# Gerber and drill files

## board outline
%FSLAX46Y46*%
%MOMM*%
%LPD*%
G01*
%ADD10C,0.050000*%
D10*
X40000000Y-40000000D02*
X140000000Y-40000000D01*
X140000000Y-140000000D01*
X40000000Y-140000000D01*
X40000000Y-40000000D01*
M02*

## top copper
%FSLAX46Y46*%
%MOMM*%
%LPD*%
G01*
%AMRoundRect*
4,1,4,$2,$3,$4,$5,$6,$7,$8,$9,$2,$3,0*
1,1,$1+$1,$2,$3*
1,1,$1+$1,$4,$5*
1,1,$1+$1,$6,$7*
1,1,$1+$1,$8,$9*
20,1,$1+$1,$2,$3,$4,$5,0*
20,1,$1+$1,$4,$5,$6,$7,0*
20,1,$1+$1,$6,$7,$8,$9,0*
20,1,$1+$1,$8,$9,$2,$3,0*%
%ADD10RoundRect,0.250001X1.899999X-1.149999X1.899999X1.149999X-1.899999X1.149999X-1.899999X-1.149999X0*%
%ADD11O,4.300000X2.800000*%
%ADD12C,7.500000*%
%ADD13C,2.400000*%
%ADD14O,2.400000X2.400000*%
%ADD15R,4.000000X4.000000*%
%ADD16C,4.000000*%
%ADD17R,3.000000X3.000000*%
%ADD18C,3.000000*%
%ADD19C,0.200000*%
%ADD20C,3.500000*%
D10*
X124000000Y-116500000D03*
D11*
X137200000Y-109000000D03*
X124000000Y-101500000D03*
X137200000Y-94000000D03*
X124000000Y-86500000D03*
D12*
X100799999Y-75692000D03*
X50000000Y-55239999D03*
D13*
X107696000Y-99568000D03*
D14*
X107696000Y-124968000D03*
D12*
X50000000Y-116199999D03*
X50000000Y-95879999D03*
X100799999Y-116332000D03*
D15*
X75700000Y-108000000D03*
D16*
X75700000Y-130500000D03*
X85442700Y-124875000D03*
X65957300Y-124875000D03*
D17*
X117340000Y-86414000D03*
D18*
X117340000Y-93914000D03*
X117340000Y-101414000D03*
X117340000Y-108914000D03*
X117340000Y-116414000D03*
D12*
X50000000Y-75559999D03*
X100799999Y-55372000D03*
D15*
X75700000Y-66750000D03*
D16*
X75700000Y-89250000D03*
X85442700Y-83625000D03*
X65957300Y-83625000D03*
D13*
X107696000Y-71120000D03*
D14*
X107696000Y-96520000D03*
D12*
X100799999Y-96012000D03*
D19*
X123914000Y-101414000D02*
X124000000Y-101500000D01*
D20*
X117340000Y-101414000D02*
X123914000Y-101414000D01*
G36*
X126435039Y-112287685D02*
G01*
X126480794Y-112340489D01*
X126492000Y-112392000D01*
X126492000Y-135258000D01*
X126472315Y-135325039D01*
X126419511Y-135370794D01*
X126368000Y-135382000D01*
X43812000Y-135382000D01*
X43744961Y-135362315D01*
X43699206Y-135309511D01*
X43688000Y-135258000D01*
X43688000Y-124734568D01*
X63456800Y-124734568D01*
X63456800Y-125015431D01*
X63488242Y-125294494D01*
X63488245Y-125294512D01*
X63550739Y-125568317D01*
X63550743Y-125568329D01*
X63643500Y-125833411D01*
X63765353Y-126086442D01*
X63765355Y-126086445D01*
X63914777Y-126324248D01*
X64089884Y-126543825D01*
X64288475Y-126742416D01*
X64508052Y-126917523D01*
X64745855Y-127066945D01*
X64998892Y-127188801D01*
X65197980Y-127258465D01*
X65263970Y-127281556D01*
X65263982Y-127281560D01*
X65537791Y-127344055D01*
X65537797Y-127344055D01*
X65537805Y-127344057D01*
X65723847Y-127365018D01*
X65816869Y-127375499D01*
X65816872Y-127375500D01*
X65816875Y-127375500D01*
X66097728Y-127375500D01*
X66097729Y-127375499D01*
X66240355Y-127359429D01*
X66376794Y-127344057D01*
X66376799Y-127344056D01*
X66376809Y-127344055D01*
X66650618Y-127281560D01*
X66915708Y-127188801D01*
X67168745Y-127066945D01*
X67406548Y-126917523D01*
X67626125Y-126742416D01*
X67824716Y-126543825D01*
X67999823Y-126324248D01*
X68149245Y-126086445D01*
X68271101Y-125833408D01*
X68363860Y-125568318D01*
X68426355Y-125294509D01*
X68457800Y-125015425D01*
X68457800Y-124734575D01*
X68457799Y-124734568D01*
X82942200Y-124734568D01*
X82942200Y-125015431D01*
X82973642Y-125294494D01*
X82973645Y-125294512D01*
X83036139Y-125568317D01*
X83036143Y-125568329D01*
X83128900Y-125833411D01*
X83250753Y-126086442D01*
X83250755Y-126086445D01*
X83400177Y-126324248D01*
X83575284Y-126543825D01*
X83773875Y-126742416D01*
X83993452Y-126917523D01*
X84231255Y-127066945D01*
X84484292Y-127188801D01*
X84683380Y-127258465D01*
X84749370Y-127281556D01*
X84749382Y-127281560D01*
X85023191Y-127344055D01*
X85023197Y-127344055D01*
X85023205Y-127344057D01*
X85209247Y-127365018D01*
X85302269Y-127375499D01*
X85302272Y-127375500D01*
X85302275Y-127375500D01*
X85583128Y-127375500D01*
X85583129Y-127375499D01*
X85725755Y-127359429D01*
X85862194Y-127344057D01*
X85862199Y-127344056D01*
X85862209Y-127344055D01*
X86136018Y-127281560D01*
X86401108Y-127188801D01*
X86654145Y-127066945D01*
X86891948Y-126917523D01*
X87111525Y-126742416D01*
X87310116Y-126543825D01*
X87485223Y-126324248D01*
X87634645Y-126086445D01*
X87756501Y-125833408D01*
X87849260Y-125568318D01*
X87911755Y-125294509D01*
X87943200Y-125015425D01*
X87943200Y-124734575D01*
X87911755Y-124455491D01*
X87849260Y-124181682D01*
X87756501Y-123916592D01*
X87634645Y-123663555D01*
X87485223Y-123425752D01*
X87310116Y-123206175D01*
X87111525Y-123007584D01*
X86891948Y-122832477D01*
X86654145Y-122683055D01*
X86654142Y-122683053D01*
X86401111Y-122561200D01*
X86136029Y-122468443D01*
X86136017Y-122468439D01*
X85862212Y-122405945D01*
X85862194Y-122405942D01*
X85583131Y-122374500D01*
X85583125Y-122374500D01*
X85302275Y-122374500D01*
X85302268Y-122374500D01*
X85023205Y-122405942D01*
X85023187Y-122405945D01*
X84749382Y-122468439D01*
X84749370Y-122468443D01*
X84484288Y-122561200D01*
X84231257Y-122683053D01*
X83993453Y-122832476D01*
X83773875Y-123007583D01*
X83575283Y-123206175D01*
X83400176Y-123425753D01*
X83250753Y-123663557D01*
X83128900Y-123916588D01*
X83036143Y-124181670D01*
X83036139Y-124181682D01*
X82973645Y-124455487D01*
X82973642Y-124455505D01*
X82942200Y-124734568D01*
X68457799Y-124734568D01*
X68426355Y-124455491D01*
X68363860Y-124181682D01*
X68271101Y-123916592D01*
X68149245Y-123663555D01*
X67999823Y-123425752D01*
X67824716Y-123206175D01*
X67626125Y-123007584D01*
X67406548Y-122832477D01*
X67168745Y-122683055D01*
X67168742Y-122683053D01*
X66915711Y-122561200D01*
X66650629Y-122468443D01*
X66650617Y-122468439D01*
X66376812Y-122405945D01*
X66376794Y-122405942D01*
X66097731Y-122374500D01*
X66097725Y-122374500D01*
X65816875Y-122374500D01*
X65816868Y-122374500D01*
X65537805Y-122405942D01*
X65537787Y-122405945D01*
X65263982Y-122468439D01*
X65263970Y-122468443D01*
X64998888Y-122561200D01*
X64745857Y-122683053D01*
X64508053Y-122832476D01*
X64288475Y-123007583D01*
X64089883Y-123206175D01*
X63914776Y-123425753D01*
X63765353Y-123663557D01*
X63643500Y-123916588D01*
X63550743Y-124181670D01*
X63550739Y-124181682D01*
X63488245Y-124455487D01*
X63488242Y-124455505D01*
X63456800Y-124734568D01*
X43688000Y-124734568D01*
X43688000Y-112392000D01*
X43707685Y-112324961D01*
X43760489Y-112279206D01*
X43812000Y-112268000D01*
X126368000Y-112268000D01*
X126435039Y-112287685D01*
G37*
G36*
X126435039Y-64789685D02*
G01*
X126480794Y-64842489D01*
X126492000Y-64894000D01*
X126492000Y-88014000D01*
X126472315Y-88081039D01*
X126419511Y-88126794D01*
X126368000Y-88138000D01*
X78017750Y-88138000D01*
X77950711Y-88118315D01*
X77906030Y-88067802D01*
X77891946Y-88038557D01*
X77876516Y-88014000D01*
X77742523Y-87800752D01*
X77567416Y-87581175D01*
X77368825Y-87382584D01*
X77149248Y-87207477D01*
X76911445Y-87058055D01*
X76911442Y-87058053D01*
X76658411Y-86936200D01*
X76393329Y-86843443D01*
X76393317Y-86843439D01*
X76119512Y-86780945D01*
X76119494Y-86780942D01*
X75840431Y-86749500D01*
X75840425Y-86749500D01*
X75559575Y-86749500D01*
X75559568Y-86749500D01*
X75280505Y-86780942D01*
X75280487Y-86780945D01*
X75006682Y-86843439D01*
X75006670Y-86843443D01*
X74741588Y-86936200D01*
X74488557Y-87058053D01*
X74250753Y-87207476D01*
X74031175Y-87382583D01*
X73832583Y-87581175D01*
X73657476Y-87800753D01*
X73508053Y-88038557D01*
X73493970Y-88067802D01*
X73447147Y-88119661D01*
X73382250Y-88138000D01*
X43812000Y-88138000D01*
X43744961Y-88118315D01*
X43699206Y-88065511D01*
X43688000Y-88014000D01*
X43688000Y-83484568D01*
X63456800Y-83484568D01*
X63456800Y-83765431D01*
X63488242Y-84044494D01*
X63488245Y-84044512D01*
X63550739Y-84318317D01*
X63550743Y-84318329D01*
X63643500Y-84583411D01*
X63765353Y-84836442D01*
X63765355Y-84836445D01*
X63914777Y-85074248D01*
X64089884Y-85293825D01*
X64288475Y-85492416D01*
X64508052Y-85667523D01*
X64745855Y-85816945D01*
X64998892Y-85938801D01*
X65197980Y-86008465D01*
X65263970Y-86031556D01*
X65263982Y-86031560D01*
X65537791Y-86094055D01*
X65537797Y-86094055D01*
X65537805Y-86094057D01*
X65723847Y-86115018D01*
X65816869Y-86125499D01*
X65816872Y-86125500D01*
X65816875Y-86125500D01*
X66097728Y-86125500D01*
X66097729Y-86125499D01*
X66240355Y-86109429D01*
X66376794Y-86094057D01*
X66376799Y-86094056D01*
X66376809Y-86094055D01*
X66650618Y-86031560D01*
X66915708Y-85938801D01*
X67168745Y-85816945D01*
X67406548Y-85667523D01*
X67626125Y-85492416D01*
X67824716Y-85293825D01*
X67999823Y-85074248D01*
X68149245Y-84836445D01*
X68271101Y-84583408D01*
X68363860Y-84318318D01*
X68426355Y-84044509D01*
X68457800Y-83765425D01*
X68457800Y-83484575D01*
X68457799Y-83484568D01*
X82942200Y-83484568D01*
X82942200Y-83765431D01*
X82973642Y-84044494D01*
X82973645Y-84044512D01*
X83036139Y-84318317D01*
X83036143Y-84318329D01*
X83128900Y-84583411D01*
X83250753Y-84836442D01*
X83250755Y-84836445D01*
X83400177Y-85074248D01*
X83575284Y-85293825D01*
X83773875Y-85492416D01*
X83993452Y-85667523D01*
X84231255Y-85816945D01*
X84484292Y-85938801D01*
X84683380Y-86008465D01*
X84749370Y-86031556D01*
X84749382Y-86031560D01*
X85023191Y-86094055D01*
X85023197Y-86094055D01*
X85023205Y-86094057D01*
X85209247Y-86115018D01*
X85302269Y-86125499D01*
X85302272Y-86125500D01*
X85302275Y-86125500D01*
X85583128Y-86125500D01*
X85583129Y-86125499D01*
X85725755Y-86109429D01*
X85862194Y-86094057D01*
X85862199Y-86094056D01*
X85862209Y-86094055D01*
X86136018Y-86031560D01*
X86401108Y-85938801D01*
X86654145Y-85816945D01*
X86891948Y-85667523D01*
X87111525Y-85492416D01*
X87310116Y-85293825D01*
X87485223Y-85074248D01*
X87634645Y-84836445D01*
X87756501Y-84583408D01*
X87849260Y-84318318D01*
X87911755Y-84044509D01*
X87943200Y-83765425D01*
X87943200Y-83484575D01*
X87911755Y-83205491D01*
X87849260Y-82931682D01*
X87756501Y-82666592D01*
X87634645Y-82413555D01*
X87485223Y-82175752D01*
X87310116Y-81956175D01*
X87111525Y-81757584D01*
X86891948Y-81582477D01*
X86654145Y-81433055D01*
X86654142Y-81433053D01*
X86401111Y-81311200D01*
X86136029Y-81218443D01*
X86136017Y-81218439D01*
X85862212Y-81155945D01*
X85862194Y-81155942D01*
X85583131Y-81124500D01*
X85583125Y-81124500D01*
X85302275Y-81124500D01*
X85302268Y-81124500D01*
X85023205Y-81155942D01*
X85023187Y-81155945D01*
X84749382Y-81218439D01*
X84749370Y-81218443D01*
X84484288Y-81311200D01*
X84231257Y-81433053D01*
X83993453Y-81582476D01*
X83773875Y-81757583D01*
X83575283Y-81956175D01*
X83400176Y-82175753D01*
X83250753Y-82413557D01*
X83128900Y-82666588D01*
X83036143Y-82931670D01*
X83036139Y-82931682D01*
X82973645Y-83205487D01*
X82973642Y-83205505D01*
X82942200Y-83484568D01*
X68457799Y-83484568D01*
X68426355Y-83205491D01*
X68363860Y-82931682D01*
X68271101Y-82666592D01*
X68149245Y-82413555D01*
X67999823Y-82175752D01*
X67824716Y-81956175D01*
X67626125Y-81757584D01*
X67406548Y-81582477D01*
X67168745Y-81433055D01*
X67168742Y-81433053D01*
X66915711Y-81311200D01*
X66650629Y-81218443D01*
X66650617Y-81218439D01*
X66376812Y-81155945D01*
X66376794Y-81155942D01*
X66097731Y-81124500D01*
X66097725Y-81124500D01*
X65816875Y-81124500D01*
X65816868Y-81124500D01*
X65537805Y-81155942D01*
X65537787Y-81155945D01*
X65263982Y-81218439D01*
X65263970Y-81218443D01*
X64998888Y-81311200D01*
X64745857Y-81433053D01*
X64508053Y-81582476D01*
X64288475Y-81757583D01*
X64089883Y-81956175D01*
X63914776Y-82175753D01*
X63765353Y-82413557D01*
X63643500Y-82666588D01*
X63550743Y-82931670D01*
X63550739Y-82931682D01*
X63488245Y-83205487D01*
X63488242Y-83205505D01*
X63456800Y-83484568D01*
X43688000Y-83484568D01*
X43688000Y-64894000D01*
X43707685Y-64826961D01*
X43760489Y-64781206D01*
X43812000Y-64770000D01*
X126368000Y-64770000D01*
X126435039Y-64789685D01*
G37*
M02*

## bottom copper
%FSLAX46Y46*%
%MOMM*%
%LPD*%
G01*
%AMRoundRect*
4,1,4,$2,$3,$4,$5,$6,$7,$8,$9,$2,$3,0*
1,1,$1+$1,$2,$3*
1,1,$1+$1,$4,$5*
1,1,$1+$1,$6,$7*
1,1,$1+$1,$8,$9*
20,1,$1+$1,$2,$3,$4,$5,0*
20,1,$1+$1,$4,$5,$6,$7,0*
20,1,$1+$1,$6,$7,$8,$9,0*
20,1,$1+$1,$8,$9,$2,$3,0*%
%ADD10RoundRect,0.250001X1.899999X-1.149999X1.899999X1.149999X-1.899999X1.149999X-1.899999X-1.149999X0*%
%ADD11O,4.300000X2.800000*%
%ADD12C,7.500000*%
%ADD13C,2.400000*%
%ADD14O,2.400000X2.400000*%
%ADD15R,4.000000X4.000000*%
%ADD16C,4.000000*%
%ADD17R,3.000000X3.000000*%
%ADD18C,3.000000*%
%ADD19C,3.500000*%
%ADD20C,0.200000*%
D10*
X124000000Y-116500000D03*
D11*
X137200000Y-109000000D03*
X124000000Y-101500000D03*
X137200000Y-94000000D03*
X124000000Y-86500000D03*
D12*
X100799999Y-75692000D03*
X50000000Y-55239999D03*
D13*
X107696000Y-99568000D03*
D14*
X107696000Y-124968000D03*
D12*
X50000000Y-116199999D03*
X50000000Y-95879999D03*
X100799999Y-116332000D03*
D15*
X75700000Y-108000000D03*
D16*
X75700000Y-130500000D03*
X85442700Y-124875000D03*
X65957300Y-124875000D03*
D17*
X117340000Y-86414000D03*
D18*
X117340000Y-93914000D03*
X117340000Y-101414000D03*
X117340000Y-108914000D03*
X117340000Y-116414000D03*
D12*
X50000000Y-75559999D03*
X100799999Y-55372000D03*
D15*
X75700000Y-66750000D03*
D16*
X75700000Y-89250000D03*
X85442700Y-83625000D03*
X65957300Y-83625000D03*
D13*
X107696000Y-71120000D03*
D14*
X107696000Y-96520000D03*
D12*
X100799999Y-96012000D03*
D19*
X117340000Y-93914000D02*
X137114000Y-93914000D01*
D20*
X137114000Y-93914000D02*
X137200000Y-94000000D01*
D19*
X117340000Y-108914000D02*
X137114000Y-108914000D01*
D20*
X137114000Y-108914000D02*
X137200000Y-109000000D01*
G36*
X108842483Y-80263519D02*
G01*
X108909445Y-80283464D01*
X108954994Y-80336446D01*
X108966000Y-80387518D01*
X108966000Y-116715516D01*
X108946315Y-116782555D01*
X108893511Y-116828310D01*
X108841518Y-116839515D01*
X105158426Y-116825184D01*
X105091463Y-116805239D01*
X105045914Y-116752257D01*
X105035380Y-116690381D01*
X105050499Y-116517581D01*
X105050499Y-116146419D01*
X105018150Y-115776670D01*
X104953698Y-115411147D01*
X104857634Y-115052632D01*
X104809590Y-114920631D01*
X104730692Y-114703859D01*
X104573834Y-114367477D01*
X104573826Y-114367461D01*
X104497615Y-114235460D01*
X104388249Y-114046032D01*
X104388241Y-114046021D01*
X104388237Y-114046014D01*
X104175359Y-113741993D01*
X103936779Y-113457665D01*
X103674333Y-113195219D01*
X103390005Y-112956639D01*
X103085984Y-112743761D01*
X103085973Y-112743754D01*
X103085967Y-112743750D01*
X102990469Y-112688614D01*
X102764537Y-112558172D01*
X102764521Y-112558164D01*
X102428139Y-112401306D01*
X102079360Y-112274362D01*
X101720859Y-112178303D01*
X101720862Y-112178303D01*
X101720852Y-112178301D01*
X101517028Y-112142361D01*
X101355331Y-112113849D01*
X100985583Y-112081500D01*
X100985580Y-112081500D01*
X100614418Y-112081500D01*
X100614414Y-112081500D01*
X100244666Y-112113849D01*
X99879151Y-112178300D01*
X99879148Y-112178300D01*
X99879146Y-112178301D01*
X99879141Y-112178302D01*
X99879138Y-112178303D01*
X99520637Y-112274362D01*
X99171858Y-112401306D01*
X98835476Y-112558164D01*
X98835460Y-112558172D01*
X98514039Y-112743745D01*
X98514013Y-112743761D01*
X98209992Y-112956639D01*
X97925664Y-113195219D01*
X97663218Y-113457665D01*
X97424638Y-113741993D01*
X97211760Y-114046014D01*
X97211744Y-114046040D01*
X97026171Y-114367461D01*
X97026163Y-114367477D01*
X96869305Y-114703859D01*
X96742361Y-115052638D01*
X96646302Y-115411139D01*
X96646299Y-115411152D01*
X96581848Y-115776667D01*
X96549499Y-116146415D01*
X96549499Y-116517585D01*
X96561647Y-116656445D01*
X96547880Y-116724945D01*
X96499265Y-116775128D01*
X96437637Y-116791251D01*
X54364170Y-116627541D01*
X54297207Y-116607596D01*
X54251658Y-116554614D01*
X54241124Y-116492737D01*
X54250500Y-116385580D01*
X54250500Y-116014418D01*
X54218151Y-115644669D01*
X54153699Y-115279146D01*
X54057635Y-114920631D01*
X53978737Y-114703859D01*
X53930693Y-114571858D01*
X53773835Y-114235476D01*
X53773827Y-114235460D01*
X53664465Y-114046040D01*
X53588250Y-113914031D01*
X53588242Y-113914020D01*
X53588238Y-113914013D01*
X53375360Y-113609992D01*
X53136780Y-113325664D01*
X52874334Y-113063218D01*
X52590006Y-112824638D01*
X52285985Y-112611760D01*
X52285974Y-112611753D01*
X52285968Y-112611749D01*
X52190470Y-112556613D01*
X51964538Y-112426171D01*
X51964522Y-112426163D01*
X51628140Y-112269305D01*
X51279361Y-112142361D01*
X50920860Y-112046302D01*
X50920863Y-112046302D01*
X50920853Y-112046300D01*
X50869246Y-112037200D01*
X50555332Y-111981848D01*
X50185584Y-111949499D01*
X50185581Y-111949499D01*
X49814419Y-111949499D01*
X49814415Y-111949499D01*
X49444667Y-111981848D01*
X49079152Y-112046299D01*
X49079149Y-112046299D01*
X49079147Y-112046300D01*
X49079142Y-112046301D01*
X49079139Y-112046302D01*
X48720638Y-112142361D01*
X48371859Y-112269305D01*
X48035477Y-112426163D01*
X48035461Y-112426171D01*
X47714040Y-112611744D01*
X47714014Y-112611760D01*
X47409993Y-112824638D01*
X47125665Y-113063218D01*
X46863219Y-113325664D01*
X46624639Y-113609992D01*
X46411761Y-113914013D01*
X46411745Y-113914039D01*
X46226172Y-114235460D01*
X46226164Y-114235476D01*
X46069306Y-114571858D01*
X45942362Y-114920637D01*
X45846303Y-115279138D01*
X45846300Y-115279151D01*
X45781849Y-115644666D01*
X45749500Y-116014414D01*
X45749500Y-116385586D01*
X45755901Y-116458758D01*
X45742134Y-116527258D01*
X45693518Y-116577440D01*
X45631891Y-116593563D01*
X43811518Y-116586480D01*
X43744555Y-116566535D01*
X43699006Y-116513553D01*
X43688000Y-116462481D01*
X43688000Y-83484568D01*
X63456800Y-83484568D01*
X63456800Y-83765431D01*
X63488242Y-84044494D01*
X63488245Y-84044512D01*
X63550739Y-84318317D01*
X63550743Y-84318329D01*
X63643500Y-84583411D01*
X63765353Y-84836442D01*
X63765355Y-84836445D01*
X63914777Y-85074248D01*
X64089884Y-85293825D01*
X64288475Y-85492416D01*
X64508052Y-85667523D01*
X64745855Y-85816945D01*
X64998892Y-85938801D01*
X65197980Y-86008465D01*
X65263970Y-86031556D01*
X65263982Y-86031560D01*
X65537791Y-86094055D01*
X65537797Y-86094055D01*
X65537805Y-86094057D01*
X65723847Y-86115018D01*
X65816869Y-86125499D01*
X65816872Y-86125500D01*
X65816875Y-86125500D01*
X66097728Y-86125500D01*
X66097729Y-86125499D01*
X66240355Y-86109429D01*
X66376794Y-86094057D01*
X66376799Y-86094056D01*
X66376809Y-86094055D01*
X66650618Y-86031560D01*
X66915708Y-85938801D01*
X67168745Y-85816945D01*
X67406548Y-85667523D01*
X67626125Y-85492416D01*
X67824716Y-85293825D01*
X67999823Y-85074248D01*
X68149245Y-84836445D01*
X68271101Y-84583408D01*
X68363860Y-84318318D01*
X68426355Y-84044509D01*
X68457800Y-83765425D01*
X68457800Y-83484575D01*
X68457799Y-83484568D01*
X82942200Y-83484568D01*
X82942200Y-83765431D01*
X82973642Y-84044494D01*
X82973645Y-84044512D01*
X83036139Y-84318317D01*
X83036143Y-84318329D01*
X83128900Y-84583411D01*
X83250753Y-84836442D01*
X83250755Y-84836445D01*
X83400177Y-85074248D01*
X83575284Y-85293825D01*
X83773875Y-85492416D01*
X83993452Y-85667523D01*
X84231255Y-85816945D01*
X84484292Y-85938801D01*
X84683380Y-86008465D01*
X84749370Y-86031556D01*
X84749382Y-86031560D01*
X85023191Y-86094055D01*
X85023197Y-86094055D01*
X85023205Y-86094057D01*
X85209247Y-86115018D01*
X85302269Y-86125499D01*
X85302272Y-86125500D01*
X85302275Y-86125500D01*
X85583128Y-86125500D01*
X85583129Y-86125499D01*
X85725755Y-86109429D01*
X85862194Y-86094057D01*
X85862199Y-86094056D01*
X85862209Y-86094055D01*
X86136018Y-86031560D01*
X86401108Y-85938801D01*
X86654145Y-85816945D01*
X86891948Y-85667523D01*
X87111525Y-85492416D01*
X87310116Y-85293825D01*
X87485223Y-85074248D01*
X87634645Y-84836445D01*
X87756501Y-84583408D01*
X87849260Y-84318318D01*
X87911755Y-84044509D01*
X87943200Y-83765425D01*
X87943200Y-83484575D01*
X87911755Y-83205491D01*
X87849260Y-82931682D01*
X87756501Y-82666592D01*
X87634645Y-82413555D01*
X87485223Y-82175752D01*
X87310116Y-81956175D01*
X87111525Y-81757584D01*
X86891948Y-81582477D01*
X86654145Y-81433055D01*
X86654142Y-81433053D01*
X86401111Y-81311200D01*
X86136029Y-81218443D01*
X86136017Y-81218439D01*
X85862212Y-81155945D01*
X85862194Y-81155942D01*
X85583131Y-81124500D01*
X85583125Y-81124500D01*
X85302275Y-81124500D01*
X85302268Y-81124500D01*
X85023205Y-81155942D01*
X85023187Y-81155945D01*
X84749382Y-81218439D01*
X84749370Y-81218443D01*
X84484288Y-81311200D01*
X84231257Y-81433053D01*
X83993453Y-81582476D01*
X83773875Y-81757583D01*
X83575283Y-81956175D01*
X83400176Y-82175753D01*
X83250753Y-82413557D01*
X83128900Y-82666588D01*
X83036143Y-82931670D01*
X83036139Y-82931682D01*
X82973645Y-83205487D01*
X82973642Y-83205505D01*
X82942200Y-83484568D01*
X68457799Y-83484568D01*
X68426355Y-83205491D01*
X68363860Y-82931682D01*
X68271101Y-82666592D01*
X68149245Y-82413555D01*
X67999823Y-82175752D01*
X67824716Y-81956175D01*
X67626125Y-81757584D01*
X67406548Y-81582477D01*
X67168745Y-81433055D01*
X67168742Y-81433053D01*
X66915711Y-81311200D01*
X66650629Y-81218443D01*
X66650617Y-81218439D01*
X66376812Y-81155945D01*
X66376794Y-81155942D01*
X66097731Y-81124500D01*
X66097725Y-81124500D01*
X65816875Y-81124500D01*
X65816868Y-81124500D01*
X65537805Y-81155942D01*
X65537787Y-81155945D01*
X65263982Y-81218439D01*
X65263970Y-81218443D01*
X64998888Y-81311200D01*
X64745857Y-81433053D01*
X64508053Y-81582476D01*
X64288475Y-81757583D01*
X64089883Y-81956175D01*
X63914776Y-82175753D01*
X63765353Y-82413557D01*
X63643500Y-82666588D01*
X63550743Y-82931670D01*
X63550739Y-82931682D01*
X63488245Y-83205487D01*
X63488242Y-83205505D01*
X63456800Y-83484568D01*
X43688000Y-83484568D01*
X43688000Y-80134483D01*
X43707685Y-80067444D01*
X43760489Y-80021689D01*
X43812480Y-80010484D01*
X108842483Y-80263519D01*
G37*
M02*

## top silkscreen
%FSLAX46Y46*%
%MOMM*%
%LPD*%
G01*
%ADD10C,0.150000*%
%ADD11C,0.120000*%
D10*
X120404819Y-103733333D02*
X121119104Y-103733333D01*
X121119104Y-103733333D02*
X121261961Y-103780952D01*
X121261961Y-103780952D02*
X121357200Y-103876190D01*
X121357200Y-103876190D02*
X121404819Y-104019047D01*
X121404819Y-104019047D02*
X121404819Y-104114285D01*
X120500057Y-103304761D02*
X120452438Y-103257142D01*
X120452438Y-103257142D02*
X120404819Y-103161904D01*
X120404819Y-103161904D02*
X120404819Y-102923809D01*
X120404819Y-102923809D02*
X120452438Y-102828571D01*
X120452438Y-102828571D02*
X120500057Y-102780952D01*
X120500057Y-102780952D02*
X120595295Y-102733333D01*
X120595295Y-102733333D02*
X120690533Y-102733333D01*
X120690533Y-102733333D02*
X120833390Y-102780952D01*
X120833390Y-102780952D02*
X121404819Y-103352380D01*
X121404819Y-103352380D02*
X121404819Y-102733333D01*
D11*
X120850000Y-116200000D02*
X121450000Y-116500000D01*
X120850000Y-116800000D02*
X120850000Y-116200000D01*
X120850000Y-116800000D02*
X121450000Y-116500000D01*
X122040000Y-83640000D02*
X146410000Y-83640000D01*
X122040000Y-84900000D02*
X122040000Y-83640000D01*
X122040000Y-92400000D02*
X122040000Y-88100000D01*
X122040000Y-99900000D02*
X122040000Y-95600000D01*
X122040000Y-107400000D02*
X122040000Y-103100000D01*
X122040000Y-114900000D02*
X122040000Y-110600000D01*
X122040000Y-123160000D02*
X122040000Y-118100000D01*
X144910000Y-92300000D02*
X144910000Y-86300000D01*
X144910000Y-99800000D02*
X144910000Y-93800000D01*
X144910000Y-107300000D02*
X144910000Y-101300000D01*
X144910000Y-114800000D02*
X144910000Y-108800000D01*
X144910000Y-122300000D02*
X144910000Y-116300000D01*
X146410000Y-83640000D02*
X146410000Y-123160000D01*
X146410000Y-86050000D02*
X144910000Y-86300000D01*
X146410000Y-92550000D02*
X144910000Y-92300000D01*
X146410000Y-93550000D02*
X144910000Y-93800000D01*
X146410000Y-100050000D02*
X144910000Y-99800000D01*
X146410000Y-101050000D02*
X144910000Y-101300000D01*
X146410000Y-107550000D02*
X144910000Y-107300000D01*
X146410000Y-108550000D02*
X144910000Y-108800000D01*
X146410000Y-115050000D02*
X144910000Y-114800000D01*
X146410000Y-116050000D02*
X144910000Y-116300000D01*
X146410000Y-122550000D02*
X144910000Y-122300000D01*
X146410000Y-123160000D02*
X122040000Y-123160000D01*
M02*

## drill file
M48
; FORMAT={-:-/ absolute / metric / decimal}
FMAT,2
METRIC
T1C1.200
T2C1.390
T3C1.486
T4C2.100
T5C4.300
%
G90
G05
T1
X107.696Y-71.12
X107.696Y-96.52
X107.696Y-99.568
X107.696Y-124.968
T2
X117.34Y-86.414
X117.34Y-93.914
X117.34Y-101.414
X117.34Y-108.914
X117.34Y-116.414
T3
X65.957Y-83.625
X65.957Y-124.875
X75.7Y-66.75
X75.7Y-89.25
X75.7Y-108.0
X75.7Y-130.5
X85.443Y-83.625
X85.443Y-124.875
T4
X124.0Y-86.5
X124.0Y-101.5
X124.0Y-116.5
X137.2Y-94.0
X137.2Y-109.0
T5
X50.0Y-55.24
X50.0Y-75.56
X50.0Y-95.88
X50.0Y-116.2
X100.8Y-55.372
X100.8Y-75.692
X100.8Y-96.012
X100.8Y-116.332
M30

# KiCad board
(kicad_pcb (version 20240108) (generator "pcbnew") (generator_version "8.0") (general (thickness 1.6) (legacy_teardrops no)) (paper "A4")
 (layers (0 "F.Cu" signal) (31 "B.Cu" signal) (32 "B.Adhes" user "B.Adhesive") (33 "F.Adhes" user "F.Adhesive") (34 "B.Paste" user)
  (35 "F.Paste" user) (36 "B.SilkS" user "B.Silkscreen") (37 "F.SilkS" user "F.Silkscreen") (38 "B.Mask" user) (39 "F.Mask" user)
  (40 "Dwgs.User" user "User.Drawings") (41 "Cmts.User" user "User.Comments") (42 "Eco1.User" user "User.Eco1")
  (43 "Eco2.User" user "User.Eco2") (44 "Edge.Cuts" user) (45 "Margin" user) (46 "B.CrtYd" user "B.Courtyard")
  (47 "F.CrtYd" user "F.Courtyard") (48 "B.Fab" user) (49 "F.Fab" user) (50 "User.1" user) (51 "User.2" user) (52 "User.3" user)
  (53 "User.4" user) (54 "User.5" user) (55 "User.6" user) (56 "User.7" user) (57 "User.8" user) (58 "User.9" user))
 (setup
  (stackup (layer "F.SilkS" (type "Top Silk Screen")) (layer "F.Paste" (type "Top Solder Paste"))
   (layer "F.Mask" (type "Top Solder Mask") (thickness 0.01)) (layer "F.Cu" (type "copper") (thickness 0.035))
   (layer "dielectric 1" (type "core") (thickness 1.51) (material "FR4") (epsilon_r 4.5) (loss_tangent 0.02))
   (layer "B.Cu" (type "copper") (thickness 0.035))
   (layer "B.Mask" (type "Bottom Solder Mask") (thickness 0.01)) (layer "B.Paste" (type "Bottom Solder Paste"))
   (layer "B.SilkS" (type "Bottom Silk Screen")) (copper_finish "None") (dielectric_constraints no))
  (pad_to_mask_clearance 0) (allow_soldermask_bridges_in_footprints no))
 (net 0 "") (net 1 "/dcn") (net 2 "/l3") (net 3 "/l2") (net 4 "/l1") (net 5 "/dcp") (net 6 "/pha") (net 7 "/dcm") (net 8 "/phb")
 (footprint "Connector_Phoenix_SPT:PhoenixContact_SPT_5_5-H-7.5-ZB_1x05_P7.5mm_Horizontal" (layer "F.Cu") (at 124 116.5 90)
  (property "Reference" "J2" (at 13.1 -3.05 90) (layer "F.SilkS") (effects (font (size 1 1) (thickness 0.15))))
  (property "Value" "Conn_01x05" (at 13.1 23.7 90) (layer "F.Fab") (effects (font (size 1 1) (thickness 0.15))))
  (fp_line (start 0.3 -3.15) (end 0 -2.55) (stroke (width 0.12) (type solid)) (layer "F.SilkS"))
  (fp_line (start -0.3 -3.15) (end 0.3 -3.15) (stroke (width 0.12) (type solid)) (layer "F.SilkS"))
  (fp_line (start -0.3 -3.15) (end 0 -2.55) (stroke (width 0.12) (type solid)) (layer "F.SilkS"))
  (fp_line (start 32.86 -1.96) (end 32.86 22.41) (stroke (width 0.12) (type solid)) (layer "F.SilkS"))
  (fp_line (start 31.6 -1.96) (end 32.86 -1.96) (stroke (width 0.12) (type solid)) (layer "F.SilkS"))
  (fp_line (start 24.1 -1.96) (end 28.4 -1.96) (stroke (width 0.12) (type solid)) (layer "F.SilkS"))
  (fp_line (start 16.6 -1.96) (end 20.9 -1.96) (stroke (width 0.12) (type solid)) (layer "F.SilkS"))
  (fp_line (start 9.1 -1.96) (end 13.4 -1.96) (stroke (width 0.12) (type solid)) (layer "F.SilkS"))
  (fp_line (start 1.6 -1.96) (end 5.9 -1.96) (stroke (width 0.12) (type solid)) (layer "F.SilkS"))
  (fp_line (start -6.66 -1.96) (end -1.6 -1.96) (stroke (width 0.12) (type solid)) (layer "F.SilkS"))
  (fp_line (start 24.2 20.91) (end 30.2 20.91) (stroke (width 0.12) (type solid)) (layer "F.SilkS"))
  (fp_line (start 16.7 20.91) (end 22.7 20.91) (stroke (width 0.12) (type solid)) (layer "F.SilkS"))
  (fp_line (start 9.2 20.91) (end 15.2 20.91) (stroke (width 0.12) (type solid)) (layer "F.SilkS"))
  (fp_line (start 1.7 20.91) (end 7.7 20.91) (stroke (width 0.12) (type solid)) (layer "F.SilkS"))
  (fp_line (start -5.8 20.91) (end 0.2 20.91) (stroke (width 0.12) (type solid)) (layer "F.SilkS"))
  (fp_line (start 32.86 22.41) (end -6.66 22.41) (stroke (width 0.12) (type solid)) (layer "F.SilkS"))
  (fp_line (start 30.45 22.41) (end 30.2 20.91) (stroke (width 0.12) (type solid)) (layer "F.SilkS"))
  (fp_line (start 23.95 22.41) (end 24.2 20.91) (stroke (width 0.12) (type solid)) (layer "F.SilkS"))
  (fp_line (start 22.95 22.41) (end 22.7 20.91) (stroke (width 0.12) (type solid)) (layer "F.SilkS"))
  (fp_line (start 16.45 22.41) (end 16.7 20.91) (stroke (width 0.12) (type solid)) (layer "F.SilkS"))
  (fp_line (start 15.45 22.41) (end 15.2 20.91) (stroke (width 0.12) (type solid)) (layer "F.SilkS"))
  (fp_line (start 8.95 22.41) (end 9.2 20.91) (stroke (width 0.12) (type solid)) (layer "F.SilkS"))
  (fp_line (start 7.95 22.41) (end 7.7 20.91) (stroke (width 0.12) (type solid)) (layer "F.SilkS"))
  (fp_line (start 1.45 22.41) (end 1.7 20.91) (stroke (width 0.12) (type solid)) (layer "F.SilkS"))
  (fp_line (start 0.45 22.41) (end 0.2 20.91) (stroke (width 0.12) (type solid)) (layer "F.SilkS"))
  (fp_line (start -6.05 22.41) (end -5.8 20.91) (stroke (width 0.12) (type solid)) (layer "F.SilkS"))
  (fp_line (start -6.66 22.41) (end -6.66 -1.96) (stroke (width 0.12) (type solid)) (layer "F.SilkS"))
  (pad "1" thru_hole roundrect (at 0 0 90) (size 2.8 4.3) (drill 2.1) (layers "*.Cu" "*.Mask") (remove_unused_layers no)
   (roundrect_rratio 0.089286) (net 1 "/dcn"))
  (pad "2" thru_hole oval (at 7.5 13.2 90) (size 2.8 4.3) (drill 2.1) (layers "*.Cu" "*.Mask") (remove_unused_layers no) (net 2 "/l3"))
  (pad "3" thru_hole oval (at 15 0 90) (size 2.8 4.3) (drill 2.1) (layers "*.Cu" "*.Mask") (remove_unused_layers no) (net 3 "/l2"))
  (pad "4" thru_hole oval (at 22.5 13.2 90) (size 2.8 4.3) (drill 2.1) (layers "*.Cu" "*.Mask") (remove_unused_layers no) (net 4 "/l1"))
  (pad "5" thru_hole oval (at 30 0 90) (size 2.8 4.3) (drill 2.1) (layers "*.Cu" "*.Mask") (remove_unused_layers no) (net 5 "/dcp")))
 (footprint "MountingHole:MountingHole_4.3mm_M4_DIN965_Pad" (layer "B.Cu") (at 100.799999 75.692 180)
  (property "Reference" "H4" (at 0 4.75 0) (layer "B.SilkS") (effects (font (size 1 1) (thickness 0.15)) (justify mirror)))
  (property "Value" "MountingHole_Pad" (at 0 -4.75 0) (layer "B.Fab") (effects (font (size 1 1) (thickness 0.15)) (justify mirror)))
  (pad "1" thru_hole circle (at 0 0 180) (size 7.5 7.5) (drill 4.3) (layers "*.Cu" "*.Mask") (remove_unused_layers no) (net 5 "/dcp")))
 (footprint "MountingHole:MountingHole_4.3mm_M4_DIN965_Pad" (layer "B.Cu") (at 50 55.239999 180)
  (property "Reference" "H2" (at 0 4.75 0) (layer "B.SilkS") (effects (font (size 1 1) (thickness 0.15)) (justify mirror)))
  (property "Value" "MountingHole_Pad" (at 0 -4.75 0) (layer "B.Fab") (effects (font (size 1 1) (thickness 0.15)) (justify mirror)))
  (pad "1" thru_hole circle (at 0 0 180) (size 7.5 7.5) (drill 4.3) (layers "*.Cu" "*.Mask") (remove_unused_layers no) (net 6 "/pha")))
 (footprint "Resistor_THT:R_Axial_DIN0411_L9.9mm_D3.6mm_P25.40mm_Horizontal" (layer "B.Cu") (at 107.696 99.568 -90)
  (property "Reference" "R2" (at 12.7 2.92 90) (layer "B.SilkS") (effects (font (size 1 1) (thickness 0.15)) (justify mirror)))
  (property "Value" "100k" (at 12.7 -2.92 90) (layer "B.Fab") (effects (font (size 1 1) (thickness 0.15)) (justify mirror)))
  (pad "1" thru_hole circle (at 0 0 270) (size 2.4 2.4) (drill 1.2) (layers "*.Cu" "*.Mask") (remove_unused_layers no) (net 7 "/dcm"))
  (pad "2" thru_hole oval (at 25.4 0 270) (size 2.4 2.4) (drill 1.2) (layers "*.Cu" "*.Mask") (remove_unused_layers no) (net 1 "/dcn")))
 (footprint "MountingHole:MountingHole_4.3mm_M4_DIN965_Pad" (layer "B.Cu") (at 50 116.199999 180)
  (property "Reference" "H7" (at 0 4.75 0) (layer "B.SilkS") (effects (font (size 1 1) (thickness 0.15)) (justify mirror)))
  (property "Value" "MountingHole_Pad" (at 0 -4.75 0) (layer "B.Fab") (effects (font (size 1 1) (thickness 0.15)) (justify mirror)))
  (pad "1" thru_hole circle (at 0 0 180) (size 7.5 7.5) (drill 4.3) (layers "*.Cu" "*.Mask") (remove_unused_layers no) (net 1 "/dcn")))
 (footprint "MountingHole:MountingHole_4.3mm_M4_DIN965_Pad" (layer "B.Cu") (at 50 95.879999 180)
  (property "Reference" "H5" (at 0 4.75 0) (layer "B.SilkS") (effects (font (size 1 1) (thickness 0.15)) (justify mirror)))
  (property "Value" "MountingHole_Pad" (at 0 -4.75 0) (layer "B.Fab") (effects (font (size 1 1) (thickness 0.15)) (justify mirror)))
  (pad "1" thru_hole circle (at 0 0 180) (size 7.5 7.5) (drill 4.3) (layers "*.Cu" "*.Mask") (remove_unused_layers no) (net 7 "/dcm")))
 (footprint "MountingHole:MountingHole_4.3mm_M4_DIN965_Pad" (layer "B.Cu") (at 100.799999 116.332 180)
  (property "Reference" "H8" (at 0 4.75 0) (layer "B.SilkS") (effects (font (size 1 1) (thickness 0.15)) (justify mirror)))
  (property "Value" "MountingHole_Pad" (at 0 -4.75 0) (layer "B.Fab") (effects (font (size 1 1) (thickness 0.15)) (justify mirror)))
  (pad "1" thru_hole circle (at 0 0 180) (size 7.5 7.5) (drill 4.3) (layers "*.Cu" "*.Mask") (remove_unused_layers no) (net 1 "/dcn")))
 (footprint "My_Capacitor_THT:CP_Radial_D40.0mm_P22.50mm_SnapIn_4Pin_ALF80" (layer "B.Cu") (at 75.7 108 -90)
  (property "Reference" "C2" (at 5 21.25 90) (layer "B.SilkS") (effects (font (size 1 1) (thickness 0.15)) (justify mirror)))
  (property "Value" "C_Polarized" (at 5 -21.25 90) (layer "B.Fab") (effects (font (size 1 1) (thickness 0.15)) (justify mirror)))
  (pad "1" thru_hole rect (at 0 0 270) (size 4 4) (drill 1.486) (layers "*.Cu" "*.Mask") (remove_unused_layers no) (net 7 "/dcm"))
  (pad "2" thru_hole circle (at 22.5 0 270) (size 4 4) (drill 1.486) (layers "*.Cu" "*.Mask") (remove_unused_layers no) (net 1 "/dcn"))
  (pad "SH" thru_hole circle (at 16.875 -9.7427 270) (size 4 4) (drill 1.486) (layers "*.Cu" "*.Mask") (remove_unused_layers no))
  (pad "SH" thru_hole circle (at 16.875 9.7427 270) (size 4 4) (drill 1.486) (layers "*.Cu" "*.Mask") (remove_unused_layers no)))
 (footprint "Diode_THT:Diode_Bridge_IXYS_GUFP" (layer "B.Cu") (at 117.34 86.414 180)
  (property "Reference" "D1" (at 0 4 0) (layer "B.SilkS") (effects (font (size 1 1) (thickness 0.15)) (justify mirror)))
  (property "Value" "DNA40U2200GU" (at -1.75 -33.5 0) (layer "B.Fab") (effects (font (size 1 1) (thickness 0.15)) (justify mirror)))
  (pad "1" thru_hole rect (at 0 0 180) (size 3 3) (drill 1.39) (layers "*.Cu" "*.Mask") (remove_unused_layers no) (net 5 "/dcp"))
  (pad "2" thru_hole circle (at 0 -7.5 180) (size 3 3) (drill 1.39) (layers "*.Cu" "*.Mask") (remove_unused_layers no) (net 4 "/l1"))
  (pad "3" thru_hole circle (at 0 -15 180) (size 3 3) (drill 1.39) (layers "*.Cu" "*.Mask") (remove_unused_layers no) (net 3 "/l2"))
  (pad "4" thru_hole circle (at 0 -22.5 180) (size 3 3) (drill 1.39) (layers "*.Cu" "*.Mask") (remove_unused_layers no) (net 2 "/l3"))
  (pad "5" thru_hole circle (at 0 -30 180) (size 3 3) (drill 1.39) (layers "*.Cu" "*.Mask") (remove_unused_layers no) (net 1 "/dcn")))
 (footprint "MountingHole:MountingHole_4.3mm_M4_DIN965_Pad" (layer "B.Cu") (at 50 75.559999 180)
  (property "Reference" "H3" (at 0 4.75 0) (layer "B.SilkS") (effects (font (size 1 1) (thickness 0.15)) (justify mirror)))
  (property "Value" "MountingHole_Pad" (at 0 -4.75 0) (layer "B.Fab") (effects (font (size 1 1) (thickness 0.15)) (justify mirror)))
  (pad "1" thru_hole circle (at 0 0 180) (size 7.5 7.5) (drill 4.3) (layers "*.Cu" "*.Mask") (remove_unused_layers no) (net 5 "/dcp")))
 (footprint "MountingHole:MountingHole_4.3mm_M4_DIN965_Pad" (layer "B.Cu") (at 100.799999 55.372 180)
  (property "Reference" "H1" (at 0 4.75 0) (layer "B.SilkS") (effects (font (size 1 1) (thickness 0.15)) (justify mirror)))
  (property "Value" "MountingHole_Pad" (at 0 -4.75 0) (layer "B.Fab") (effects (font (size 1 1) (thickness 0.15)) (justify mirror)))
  (pad "1" thru_hole circle (at 0 0 180) (size 7.5 7.5) (drill 4.3) (layers "*.Cu" "*.Mask") (remove_unused_layers no) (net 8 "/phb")))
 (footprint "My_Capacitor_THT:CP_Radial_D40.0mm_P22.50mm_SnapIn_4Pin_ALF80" (layer "B.Cu") (at 75.7 66.75 -90)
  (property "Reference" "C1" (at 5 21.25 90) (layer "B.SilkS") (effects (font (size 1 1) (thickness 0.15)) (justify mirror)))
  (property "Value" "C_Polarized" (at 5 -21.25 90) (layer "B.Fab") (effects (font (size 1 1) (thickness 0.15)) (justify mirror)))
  (pad "1" thru_hole rect (at 0 0 270) (size 4 4) (drill 1.486) (layers "*.Cu" "*.Mask") (remove_unused_layers no) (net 5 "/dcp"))
  (pad "2" thru_hole circle (at 22.5 0 270) (size 4 4) (drill 1.486) (layers "*.Cu" "*.Mask") (remove_unused_layers no) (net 7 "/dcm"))
  (pad "SH" thru_hole circle (at 16.875 -9.7427 270) (size 4 4) (drill 1.486) (layers "*.Cu" "*.Mask") (remove_unused_layers no))
  (pad "SH" thru_hole circle (at 16.875 9.7427 270) (size 4 4) (drill 1.486) (layers "*.Cu" "*.Mask") (remove_unused_layers no)))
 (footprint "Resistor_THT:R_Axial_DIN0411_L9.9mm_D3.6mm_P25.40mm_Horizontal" (layer "B.Cu") (at 107.696 71.12 -90)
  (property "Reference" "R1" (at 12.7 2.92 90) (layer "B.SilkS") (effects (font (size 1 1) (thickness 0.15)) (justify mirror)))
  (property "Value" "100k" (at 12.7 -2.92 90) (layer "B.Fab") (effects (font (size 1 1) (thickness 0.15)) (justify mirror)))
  (pad "1" thru_hole circle (at 0 0 270) (size 2.4 2.4) (drill 1.2) (layers "*.Cu" "*.Mask") (remove_unused_layers no) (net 5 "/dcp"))
  (pad "2" thru_hole oval (at 25.4 0 270) (size 2.4 2.4) (drill 1.2) (layers "*.Cu" "*.Mask") (remove_unused_layers no) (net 7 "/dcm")))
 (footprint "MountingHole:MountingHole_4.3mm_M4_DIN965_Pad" (layer "B.Cu") (at 100.799999 96.012 180)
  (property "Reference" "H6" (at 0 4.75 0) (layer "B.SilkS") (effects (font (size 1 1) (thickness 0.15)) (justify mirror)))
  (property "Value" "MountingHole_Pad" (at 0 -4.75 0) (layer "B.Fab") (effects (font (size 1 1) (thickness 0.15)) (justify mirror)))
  (pad "1" thru_hole circle (at 0 0 180) (size 7.5 7.5) (drill 4.3) (layers "*.Cu" "*.Mask") (remove_unused_layers no) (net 7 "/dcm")))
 (gr_rect (start 40 40) (end 140 140) (stroke (width 0.05) (type default)) (fill none) (layer "Edge.Cuts"))
 (segment (start 117.34 93.914) (end 137.114 93.914) (width 3.5) (layer "B.Cu") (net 4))
 (segment (start 137.114 93.914) (end 137.2 94) (width 0.2) (layer "B.Cu") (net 4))
 (segment (start 123.914 101.414) (end 124 101.5) (width 0.2) (layer "F.Cu") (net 3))
 (segment (start 117.34 101.414) (end 123.914 101.414) (width 3.5) (layer "F.Cu") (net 3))
 (segment (start 117.34 108.914) (end 137.114 108.914) (width 3.5) (layer "B.Cu") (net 2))
 (segment (start 137.114 108.914) (end 137.2 109) (width 0.2) (layer "B.Cu") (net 2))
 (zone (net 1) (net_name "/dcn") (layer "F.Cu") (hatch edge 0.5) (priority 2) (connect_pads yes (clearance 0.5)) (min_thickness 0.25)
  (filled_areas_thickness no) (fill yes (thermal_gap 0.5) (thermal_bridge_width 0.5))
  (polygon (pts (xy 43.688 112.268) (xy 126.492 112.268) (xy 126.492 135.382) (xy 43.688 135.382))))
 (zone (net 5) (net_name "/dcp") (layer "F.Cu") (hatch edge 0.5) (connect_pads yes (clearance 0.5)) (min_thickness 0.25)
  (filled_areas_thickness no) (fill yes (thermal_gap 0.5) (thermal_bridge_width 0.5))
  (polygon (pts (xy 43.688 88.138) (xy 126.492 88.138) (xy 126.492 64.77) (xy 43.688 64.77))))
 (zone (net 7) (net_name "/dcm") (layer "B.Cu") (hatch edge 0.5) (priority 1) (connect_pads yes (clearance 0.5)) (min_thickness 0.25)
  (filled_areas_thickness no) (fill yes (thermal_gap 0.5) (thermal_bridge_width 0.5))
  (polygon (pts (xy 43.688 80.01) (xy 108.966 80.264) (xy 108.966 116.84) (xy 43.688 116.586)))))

